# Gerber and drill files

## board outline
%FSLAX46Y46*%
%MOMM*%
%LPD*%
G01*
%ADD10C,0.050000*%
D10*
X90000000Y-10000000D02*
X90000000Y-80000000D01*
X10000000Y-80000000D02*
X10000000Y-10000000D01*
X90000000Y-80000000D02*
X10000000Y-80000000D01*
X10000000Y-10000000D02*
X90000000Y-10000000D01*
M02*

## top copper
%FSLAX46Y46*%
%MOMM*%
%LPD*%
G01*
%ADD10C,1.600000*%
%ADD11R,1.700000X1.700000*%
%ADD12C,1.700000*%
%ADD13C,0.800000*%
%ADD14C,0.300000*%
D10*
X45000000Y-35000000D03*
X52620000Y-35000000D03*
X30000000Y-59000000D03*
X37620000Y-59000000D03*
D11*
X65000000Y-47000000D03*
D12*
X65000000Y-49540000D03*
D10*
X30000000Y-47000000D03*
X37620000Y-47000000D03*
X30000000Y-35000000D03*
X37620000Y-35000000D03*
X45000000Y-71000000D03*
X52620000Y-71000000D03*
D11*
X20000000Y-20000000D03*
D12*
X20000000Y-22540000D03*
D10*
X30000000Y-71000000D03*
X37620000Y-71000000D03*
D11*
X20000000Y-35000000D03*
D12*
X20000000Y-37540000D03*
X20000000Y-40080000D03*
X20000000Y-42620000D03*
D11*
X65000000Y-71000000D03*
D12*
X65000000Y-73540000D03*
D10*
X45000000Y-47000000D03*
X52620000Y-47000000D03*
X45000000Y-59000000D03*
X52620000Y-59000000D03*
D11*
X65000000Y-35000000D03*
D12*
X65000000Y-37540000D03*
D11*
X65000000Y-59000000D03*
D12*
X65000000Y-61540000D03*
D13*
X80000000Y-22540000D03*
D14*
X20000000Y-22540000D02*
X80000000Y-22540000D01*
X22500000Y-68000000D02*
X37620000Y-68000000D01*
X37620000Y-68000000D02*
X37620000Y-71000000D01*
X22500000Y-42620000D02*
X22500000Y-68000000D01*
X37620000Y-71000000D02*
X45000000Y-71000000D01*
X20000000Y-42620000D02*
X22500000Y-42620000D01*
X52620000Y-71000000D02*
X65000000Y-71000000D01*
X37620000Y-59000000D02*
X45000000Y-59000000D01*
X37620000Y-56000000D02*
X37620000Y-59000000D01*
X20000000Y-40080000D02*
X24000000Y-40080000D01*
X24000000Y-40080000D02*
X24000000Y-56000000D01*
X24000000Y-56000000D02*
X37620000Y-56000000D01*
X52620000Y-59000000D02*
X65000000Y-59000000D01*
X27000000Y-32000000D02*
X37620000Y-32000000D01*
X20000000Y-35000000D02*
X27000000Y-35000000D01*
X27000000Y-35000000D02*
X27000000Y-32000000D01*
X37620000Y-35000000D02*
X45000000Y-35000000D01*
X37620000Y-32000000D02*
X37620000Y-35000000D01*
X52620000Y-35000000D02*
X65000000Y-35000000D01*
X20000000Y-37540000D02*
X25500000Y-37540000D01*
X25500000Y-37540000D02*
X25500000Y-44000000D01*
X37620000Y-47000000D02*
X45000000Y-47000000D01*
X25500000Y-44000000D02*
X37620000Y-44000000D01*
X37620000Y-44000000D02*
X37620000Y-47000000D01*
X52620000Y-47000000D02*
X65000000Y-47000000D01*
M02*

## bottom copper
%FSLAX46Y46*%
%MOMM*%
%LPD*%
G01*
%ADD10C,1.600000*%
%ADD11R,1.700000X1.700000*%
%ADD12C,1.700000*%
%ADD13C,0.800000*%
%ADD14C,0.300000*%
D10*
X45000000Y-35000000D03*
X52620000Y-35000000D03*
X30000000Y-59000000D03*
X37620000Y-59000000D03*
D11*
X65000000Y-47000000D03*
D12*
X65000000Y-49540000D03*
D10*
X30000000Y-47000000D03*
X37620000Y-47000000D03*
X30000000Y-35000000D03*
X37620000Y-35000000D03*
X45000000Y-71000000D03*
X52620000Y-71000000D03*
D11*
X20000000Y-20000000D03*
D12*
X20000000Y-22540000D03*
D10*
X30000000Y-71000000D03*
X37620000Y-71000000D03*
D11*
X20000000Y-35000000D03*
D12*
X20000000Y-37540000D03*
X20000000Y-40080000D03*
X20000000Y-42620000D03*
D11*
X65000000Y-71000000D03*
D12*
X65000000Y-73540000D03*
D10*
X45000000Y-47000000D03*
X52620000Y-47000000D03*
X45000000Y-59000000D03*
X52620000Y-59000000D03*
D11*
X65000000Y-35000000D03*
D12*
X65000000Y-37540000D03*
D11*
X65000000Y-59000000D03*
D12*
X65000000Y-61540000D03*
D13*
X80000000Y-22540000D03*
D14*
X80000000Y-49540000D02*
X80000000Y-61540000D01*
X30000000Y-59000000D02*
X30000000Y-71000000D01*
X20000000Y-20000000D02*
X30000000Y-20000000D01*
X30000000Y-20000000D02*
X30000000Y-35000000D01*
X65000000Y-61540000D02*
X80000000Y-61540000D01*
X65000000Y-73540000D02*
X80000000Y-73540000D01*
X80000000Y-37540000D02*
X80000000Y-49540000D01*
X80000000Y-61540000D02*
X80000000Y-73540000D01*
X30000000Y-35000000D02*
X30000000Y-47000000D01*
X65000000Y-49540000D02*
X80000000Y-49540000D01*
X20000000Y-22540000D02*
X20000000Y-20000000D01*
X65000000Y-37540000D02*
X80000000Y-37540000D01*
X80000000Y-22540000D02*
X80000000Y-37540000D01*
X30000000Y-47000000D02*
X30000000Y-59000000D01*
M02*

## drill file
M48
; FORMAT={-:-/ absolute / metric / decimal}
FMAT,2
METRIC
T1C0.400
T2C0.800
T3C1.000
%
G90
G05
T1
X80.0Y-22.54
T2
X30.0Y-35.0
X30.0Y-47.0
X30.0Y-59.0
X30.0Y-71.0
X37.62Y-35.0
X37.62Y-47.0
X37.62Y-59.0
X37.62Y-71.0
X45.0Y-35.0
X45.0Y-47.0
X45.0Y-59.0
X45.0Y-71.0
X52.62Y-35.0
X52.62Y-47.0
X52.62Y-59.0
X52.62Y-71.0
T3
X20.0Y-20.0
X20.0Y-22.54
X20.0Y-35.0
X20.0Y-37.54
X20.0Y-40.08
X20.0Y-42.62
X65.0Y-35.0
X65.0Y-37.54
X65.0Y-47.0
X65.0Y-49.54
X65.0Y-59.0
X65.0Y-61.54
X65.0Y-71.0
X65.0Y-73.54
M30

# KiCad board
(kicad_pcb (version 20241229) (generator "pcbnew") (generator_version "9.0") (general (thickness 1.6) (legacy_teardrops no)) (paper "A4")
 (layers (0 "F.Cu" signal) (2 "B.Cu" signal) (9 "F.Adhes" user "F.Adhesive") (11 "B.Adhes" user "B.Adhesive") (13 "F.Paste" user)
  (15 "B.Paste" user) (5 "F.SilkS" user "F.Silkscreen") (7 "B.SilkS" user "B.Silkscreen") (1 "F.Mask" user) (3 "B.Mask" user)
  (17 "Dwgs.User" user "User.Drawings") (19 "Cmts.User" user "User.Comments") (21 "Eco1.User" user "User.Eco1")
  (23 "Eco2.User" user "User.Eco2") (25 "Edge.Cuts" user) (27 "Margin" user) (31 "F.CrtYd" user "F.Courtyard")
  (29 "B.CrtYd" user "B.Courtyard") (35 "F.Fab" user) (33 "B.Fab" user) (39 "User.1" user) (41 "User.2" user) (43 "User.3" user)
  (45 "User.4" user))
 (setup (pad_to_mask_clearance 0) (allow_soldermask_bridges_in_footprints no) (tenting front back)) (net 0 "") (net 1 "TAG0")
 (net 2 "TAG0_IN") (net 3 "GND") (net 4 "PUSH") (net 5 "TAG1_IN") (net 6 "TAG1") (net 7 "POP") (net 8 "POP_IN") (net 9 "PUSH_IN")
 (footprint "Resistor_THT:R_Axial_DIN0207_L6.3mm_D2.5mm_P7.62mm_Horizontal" (layer "F.Cu") (at 45 35)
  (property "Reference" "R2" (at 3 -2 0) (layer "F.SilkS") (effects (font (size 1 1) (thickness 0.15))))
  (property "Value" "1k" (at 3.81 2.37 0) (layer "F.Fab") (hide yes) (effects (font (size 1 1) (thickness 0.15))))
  (pad "1" thru_hole circle (at 0 0) (size 1.6 1.6) (drill 0.8) (layers "*.Cu" "*.Mask") (remove_unused_layers no) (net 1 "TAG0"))
  (pad "2" thru_hole circle (at 7.62 0) (size 1.6 1.6) (drill 0.8) (layers "*.Cu" "*.Mask") (remove_unused_layers no) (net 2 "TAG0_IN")))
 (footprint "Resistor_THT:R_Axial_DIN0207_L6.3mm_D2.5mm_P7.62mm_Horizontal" (layer "F.Cu") (at 30 59)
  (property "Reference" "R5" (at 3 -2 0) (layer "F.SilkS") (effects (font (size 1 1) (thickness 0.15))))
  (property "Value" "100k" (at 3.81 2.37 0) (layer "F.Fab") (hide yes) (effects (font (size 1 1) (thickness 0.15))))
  (pad "1" thru_hole circle (at 0 0) (size 1.6 1.6) (drill 0.8) (layers "*.Cu" "*.Mask") (remove_unused_layers no) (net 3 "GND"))
  (pad "2" thru_hole circle (at 7.62 0) (size 1.6 1.6) (drill 0.8) (layers "*.Cu" "*.Mask") (remove_unused_layers no) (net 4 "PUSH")))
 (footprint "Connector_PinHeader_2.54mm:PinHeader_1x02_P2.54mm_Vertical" (layer "F.Cu") (at 65 47)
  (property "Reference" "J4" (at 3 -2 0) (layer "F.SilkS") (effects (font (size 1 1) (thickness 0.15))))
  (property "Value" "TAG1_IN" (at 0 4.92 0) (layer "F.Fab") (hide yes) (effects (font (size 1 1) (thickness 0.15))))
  (pad "1" thru_hole rect (at 0 0) (size 1.7 1.7) (drill 1) (layers "*.Cu" "*.Mask") (remove_unused_layers no) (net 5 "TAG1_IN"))
  (pad "2" thru_hole circle (at 0 2.54) (size 1.7 1.7) (drill 1) (layers "*.Cu" "*.Mask") (remove_unused_layers no) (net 3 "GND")))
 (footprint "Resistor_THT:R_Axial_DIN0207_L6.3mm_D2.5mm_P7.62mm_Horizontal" (layer "F.Cu") (at 30 47)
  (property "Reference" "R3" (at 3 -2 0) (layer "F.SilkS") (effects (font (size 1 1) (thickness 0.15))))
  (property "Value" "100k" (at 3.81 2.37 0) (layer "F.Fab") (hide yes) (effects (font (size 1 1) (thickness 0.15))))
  (pad "1" thru_hole circle (at 0 0) (size 1.6 1.6) (drill 0.8) (layers "*.Cu" "*.Mask") (remove_unused_layers no) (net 3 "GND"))
  (pad "2" thru_hole circle (at 7.62 0) (size 1.6 1.6) (drill 0.8) (layers "*.Cu" "*.Mask") (remove_unused_layers no) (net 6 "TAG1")))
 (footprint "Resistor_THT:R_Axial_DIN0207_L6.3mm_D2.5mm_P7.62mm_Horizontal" (layer "F.Cu") (at 30 35)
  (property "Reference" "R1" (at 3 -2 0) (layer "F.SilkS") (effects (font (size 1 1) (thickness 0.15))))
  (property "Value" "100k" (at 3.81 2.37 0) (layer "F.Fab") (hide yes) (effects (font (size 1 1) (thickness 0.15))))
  (pad "1" thru_hole circle (at 0 0) (size 1.6 1.6) (drill 0.8) (layers "*.Cu" "*.Mask") (remove_unused_layers no) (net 3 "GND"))
  (pad "2" thru_hole circle (at 7.62 0) (size 1.6 1.6) (drill 0.8) (layers "*.Cu" "*.Mask") (remove_unused_layers no) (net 1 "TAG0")))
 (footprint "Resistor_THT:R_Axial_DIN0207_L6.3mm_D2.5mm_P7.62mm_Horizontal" (layer "F.Cu") (at 45 71)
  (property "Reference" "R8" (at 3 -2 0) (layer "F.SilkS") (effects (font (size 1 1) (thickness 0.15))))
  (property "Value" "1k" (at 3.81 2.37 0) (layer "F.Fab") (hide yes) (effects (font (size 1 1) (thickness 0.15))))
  (pad "1" thru_hole circle (at 0 0) (size 1.6 1.6) (drill 0.8) (layers "*.Cu" "*.Mask") (remove_unused_layers no) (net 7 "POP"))
  (pad "2" thru_hole circle (at 7.62 0) (size 1.6 1.6) (drill 0.8) (layers "*.Cu" "*.Mask") (remove_unused_layers no) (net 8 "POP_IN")))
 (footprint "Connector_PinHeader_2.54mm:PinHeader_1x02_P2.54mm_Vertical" (layer "F.Cu") (at 20 20)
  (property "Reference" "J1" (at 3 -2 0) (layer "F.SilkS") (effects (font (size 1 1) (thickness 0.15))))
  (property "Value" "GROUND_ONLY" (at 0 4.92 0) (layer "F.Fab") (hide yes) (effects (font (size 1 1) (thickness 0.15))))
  (pad "1" thru_hole rect (at 0 0) (size 1.7 1.7) (drill 1) (layers "*.Cu" "*.Mask") (remove_unused_layers no) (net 3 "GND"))
  (pad "2" thru_hole circle (at 0 2.54) (size 1.7 1.7) (drill 1) (layers "*.Cu" "*.Mask") (remove_unused_layers no) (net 3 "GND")))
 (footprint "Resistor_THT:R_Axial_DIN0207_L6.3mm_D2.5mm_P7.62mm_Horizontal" (layer "F.Cu") (at 30 71)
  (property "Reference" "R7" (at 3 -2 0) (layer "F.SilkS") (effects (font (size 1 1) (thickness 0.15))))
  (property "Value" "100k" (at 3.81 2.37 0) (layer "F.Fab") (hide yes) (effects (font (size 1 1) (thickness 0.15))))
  (pad "1" thru_hole circle (at 0 0) (size 1.6 1.6) (drill 0.8) (layers "*.Cu" "*.Mask") (remove_unused_layers no) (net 3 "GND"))
  (pad "2" thru_hole circle (at 7.62 0) (size 1.6 1.6) (drill 0.8) (layers "*.Cu" "*.Mask") (remove_unused_layers no) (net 7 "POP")))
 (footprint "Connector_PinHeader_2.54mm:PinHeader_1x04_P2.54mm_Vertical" (layer "F.Cu") (at 20 35)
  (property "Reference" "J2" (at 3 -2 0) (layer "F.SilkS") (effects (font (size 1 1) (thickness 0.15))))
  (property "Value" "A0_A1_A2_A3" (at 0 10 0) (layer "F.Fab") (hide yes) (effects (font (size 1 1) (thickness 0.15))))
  (pad "1" thru_hole rect (at 0 0) (size 1.7 1.7) (drill 1) (layers "*.Cu" "*.Mask") (remove_unused_layers no) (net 1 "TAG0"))
  (pad "2" thru_hole circle (at 0 2.54) (size 1.7 1.7) (drill 1) (layers "*.Cu" "*.Mask") (remove_unused_layers no) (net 6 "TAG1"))
  (pad "3" thru_hole circle (at 0 5.08) (size 1.7 1.7) (drill 1) (layers "*.Cu" "*.Mask") (remove_unused_layers no) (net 4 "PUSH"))
  (pad "4" thru_hole circle (at 0 7.62) (size 1.7 1.7) (drill 1) (layers "*.Cu" "*.Mask") (remove_unused_layers no) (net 7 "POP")))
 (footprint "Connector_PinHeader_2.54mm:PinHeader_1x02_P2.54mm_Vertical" (layer "F.Cu") (at 65 71)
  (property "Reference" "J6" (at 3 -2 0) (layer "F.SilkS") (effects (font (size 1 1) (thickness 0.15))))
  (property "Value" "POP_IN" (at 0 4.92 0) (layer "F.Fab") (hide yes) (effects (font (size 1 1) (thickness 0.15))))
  (pad "1" thru_hole rect (at 0 0) (size 1.7 1.7) (drill 1) (layers "*.Cu" "*.Mask") (remove_unused_layers no) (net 8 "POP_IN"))
  (pad "2" thru_hole circle (at 0 2.54) (size 1.7 1.7) (drill 1) (layers "*.Cu" "*.Mask") (remove_unused_layers no) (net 3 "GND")))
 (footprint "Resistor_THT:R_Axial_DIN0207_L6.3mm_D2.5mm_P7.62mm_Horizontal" (layer "F.Cu") (at 45 47)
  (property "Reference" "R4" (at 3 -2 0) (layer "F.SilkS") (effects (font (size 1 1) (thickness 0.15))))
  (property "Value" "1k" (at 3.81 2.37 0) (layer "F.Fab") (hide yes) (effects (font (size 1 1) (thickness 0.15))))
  (pad "1" thru_hole circle (at 0 0) (size 1.6 1.6) (drill 0.8) (layers "*.Cu" "*.Mask") (remove_unused_layers no) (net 6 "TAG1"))
  (pad "2" thru_hole circle (at 7.62 0) (size 1.6 1.6) (drill 0.8) (layers "*.Cu" "*.Mask") (remove_unused_layers no) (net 5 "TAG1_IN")))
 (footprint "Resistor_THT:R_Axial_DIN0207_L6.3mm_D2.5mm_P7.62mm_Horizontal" (layer "F.Cu") (at 45 59)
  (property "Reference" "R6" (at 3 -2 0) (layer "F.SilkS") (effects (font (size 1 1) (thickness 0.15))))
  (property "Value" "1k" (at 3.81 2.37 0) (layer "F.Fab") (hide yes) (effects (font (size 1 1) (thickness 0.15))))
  (pad "1" thru_hole circle (at 0 0) (size 1.6 1.6) (drill 0.8) (layers "*.Cu" "*.Mask") (remove_unused_layers no) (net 4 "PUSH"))
  (pad "2" thru_hole circle (at 7.62 0) (size 1.6 1.6) (drill 0.8) (layers "*.Cu" "*.Mask") (remove_unused_layers no) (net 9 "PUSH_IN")))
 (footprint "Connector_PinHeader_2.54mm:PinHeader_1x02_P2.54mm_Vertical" (layer "F.Cu") (at 65 35)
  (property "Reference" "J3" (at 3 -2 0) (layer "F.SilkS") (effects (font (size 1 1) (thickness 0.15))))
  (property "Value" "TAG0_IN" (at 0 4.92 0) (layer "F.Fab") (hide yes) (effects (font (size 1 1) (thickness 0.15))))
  (pad "1" thru_hole rect (at 0 0) (size 1.7 1.7) (drill 1) (layers "*.Cu" "*.Mask") (remove_unused_layers no) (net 2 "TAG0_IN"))
  (pad "2" thru_hole circle (at 0 2.54) (size 1.7 1.7) (drill 1) (layers "*.Cu" "*.Mask") (remove_unused_layers no) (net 3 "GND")))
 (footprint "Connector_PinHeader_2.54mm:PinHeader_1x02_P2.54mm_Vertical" (layer "F.Cu") (at 65 59)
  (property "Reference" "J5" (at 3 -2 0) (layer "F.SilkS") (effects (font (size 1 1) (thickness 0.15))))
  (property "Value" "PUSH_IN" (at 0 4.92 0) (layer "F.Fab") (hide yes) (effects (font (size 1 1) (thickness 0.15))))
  (pad "1" thru_hole rect (at 0 0) (size 1.7 1.7) (drill 1) (layers "*.Cu" "*.Mask") (remove_unused_layers no) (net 9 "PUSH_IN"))
  (pad "2" thru_hole circle (at 0 2.54) (size 1.7 1.7) (drill 1) (layers "*.Cu" "*.Mask") (remove_unused_layers no) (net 3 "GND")))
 (gr_line (start 90 10) (end 90 80) (stroke (width 0.05) (type default)) (layer "Edge.Cuts"))
 (gr_line (start 10 80) (end 10 10) (stroke (width 0.05) (type default)) (layer "Edge.Cuts"))
 (gr_line (start 90 80) (end 10 80) (stroke (width 0.05) (type default)) (layer "Edge.Cuts"))
 (gr_line (start 10 10) (end 90 10) (stroke (width 0.05) (type default)) (layer "Edge.Cuts"))
 (segment (start 20 22.54) (end 80 22.54) (width 0.3) (layer "F.Cu") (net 3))
 (via (at 80 22.54) (size 0.8) (drill 0.4) (layers "F.Cu" "B.Cu") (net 3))
 (segment (start 80 49.54) (end 80 61.54) (width 0.3) (layer "B.Cu") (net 3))
 (segment (start 30 59) (end 30 71) (width 0.3) (layer "B.Cu") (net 3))
 (segment (start 20 20) (end 30 20) (width 0.3) (layer "B.Cu") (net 3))
 (segment (start 30 20) (end 30 35) (width 0.3) (layer "B.Cu") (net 3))
 (segment (start 65 61.54) (end 80 61.54) (width 0.3) (layer "B.Cu") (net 3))
 (segment (start 65 73.54) (end 80 73.54) (width 0.3) (layer "B.Cu") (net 3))
 (segment (start 80 37.54) (end 80 49.54) (width 0.3) (layer "B.Cu") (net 3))
 (segment (start 80 61.54) (end 80 73.54) (width 0.3) (layer "B.Cu") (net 3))
 (segment (start 30 35) (end 30 47) (width 0.3) (layer "B.Cu") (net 3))
 (segment (start 65 49.54) (end 80 49.54) (width 0.3) (layer "B.Cu") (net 3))
 (segment (start 20 22.54) (end 20 20) (width 0.3) (layer "B.Cu") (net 3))
 (segment (start 65 37.54) (end 80 37.54) (width 0.3) (layer "B.Cu") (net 3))
 (segment (start 80 22.54) (end 80 37.54) (width 0.3) (layer "B.Cu") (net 3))
 (segment (start 30 47) (end 30 59) (width 0.3) (layer "B.Cu") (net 3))
 (segment (start 22.5 68) (end 37.62 68) (width 0.3) (layer "F.Cu") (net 7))
 (segment (start 37.62 68) (end 37.62 71) (width 0.3) (layer "F.Cu") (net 7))
 (segment (start 22.5 42.62) (end 22.5 68) (width 0.3) (layer "F.Cu") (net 7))
 (segment (start 37.62 71) (end 45 71) (width 0.3) (layer "F.Cu") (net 7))
 (segment (start 20 42.62) (end 22.5 42.62) (width 0.3) (layer "F.Cu") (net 7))
 (segment (start 52.62 71) (end 65 71) (width 0.3) (layer "F.Cu") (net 8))
 (segment (start 37.62 59) (end 45 59) (width 0.3) (layer "F.Cu") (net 4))
 (segment (start 37.62 56) (end 37.62 59) (width 0.3) (layer "F.Cu") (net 4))
 (segment (start 20 40.08) (end 24 40.08) (width 0.3) (layer "F.Cu") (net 4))
 (segment (start 24 40.08) (end 24 56) (width 0.3) (layer "F.Cu") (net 4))
 (segment (start 24 56) (end 37.62 56) (width 0.3) (layer "F.Cu") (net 4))
 (segment (start 52.62 59) (end 65 59) (width 0.3) (layer "F.Cu") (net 9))
 (segment (start 27 32) (end 37.62 32) (width 0.3) (layer "F.Cu") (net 1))
 (segment (start 20 35) (end 27 35) (width 0.3) (layer "F.Cu") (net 1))
 (segment (start 27 35) (end 27 32) (width 0.3) (layer "F.Cu") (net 1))
 (segment (start 37.62 35) (end 45 35) (width 0.3) (layer "F.Cu") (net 1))
 (segment (start 37.62 32) (end 37.62 35) (width 0.3) (layer "F.Cu") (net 1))
 (segment (start 52.62 35) (end 65 35) (width 0.3) (layer "F.Cu") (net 2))
 (segment (start 20 37.54) (end 25.5 37.54) (width 0.3) (layer "F.Cu") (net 6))
 (segment (start 25.5 37.54) (end 25.5 44) (width 0.3) (layer "F.Cu") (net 6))
 (segment (start 37.62 47) (end 45 47) (width 0.3) (layer "F.Cu") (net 6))
 (segment (start 25.5 44) (end 37.62 44) (width 0.3) (layer "F.Cu") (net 6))
 (segment (start 37.62 44) (end 37.62 47) (width 0.3) (layer "F.Cu") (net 6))
 (segment (start 52.62 47) (end 65 47) (width 0.3) (layer "F.Cu") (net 5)))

